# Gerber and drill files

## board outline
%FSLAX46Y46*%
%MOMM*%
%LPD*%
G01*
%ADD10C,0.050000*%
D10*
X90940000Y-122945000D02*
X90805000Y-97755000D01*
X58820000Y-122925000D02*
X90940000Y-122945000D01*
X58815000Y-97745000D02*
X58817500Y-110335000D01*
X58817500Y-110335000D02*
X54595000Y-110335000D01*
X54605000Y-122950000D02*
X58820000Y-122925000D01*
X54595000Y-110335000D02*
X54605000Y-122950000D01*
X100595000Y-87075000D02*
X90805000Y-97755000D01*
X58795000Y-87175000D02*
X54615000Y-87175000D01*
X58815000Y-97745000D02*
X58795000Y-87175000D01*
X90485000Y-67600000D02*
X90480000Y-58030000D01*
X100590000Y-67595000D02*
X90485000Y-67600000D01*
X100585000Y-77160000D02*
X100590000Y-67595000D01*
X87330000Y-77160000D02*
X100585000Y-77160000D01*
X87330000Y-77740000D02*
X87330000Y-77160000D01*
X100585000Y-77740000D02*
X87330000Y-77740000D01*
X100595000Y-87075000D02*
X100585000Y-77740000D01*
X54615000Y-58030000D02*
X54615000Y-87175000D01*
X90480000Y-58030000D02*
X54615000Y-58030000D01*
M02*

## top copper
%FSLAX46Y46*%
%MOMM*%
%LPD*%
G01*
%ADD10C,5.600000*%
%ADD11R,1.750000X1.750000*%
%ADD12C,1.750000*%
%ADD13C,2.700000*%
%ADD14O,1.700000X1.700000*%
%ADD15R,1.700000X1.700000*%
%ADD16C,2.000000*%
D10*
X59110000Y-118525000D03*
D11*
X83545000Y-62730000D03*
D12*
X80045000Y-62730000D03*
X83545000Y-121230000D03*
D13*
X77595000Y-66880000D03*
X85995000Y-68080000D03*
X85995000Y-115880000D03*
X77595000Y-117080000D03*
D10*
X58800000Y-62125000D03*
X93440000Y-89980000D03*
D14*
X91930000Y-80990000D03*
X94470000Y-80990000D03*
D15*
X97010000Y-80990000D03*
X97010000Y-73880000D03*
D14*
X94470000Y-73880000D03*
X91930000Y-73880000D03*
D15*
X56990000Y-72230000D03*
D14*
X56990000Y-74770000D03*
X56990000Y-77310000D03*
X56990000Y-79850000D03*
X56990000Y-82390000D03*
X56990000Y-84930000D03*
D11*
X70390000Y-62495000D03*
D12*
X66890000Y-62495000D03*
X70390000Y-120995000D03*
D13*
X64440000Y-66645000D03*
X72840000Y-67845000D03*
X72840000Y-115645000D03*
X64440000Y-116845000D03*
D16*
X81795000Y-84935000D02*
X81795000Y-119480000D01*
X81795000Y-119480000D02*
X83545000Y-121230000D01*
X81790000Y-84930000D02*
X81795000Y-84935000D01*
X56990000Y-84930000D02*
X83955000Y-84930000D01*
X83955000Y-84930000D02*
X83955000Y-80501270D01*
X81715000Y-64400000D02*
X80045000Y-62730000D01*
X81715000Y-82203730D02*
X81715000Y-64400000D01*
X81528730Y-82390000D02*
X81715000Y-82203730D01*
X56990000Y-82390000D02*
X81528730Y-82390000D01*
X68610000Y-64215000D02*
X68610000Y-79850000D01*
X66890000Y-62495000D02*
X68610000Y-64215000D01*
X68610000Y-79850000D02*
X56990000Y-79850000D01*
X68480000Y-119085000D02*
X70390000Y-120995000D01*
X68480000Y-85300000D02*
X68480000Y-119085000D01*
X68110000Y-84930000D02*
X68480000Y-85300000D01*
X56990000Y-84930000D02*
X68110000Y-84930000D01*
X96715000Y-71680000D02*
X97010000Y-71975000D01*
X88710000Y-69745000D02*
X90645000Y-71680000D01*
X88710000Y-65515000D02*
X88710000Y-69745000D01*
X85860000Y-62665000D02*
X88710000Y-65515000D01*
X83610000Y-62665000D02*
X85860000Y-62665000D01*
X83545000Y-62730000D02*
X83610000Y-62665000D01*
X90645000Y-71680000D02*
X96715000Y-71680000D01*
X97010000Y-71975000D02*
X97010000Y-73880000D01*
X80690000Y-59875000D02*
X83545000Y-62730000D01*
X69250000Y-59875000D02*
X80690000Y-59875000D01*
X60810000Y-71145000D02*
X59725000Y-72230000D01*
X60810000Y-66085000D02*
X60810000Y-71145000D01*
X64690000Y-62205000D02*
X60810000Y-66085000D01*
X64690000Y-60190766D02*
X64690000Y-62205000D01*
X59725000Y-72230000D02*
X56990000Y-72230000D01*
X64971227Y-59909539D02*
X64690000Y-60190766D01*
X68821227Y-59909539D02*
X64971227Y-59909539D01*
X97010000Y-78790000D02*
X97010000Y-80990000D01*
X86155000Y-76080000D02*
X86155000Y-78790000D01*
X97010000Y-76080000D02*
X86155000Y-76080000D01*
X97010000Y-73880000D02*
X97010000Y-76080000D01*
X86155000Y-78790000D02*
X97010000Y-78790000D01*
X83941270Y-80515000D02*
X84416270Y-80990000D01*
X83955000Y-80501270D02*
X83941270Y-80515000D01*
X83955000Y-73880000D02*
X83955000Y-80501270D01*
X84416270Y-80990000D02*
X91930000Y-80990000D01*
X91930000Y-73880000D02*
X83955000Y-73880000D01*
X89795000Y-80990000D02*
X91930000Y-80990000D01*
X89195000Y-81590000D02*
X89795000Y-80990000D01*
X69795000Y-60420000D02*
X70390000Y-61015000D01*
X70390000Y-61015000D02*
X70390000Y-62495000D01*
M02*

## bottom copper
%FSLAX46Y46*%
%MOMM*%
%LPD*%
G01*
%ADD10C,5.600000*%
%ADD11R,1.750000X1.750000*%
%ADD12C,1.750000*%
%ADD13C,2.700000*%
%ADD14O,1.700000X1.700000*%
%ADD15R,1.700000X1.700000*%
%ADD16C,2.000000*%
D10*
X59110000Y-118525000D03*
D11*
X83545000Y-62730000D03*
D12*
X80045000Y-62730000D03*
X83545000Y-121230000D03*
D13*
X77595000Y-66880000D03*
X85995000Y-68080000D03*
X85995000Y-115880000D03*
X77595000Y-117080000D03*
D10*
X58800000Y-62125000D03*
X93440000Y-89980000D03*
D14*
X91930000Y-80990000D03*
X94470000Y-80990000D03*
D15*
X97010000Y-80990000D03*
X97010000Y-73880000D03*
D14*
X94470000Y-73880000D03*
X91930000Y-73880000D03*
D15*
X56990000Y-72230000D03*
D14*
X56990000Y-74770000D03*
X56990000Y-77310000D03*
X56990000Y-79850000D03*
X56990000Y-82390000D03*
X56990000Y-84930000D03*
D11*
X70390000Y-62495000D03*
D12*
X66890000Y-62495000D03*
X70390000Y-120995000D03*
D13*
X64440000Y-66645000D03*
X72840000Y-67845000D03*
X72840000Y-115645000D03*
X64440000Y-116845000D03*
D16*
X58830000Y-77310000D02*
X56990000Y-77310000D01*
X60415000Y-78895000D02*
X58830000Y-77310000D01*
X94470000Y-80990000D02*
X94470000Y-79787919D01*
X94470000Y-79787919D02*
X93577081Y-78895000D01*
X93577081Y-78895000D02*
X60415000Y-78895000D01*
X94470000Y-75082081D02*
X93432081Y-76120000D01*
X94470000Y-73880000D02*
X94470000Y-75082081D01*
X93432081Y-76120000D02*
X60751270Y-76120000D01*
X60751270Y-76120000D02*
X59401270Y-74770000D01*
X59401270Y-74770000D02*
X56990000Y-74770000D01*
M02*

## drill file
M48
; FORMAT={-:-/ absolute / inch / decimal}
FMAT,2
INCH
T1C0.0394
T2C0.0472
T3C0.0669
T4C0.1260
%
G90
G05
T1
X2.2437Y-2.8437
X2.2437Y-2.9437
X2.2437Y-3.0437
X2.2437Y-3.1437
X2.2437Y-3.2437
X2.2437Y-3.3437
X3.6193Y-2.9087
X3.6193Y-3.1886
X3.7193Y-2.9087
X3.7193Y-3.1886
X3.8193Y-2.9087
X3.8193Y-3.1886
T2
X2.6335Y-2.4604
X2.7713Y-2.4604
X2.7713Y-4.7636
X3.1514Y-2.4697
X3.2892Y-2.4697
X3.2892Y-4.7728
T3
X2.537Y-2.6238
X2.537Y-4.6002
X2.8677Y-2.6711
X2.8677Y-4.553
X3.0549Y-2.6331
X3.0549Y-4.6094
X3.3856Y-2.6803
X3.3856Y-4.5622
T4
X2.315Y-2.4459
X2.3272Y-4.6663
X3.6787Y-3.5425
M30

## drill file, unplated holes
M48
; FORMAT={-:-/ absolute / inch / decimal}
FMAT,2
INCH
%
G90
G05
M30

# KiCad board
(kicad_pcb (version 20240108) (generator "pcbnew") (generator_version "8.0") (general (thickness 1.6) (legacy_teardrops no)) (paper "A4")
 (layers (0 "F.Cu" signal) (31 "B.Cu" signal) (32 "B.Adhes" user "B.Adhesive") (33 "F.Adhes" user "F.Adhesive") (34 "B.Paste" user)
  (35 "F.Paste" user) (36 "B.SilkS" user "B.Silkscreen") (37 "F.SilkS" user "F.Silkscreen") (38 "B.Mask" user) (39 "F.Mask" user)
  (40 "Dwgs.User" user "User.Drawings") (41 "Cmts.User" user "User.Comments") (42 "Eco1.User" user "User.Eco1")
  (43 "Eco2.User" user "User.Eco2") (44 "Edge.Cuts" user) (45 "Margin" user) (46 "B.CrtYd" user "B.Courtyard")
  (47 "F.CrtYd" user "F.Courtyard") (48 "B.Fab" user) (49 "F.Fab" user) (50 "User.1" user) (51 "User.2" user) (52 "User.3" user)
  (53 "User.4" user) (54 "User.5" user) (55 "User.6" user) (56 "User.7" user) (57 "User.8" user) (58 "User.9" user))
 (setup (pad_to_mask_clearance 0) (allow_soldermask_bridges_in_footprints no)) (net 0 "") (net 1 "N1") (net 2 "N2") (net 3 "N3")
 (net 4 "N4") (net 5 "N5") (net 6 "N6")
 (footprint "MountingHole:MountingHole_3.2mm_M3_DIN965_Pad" (layer "F.Cu") (at 93.44 89.98)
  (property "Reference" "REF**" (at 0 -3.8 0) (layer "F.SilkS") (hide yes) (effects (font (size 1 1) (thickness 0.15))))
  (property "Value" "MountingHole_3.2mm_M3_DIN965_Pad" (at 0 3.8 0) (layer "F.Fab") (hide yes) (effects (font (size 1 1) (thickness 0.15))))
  (pad "1" thru_hole circle (at 0 0) (size 5.6 5.6) (drill 3.2) (layers "*.Cu" "*.Mask") (remove_unused_layers no)))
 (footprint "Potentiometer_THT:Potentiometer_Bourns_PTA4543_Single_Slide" (layer "F.Cu") (at 83.545 62.73 -90)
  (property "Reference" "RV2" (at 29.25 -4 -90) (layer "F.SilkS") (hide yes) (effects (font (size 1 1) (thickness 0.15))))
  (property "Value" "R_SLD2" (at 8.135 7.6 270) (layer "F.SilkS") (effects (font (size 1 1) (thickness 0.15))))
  (pad "1" thru_hole rect (at 0 0 270) (size 1.75 1.75) (drill 1.2) (layers "*.Cu" "*.Mask") (remove_unused_layers no) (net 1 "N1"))
  (pad "2" thru_hole circle (at 0 3.5 270) (size 1.75 1.75) (drill 1.2) (layers "*.Cu" "*.Mask") (remove_unused_layers no) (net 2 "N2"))
  (pad "3" thru_hole circle (at 58.5 0 270) (size 1.75 1.75) (drill 1.2) (layers "*.Cu" "*.Mask") (remove_unused_layers no) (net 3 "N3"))
  (pad "MP" thru_hole circle (at 4.15 5.95 270) (size 2.7 2.7) (drill 1.7) (layers "*.Cu" "*.Mask") (remove_unused_layers no))
  (pad "MP" thru_hole circle (at 5.35 -2.45 270) (size 2.7 2.7) (drill 1.7) (layers "*.Cu" "*.Mask") (remove_unused_layers no))
  (pad "MP" thru_hole circle (at 53.15 -2.45 270) (size 2.7 2.7) (drill 1.7) (layers "*.Cu" "*.Mask") (remove_unused_layers no))
  (pad "MP" thru_hole circle (at 54.35 5.95 270) (size 2.7 2.7) (drill 1.7) (layers "*.Cu" "*.Mask") (remove_unused_layers no)))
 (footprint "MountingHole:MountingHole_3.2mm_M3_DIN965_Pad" (layer "F.Cu") (at 58.8 62.125)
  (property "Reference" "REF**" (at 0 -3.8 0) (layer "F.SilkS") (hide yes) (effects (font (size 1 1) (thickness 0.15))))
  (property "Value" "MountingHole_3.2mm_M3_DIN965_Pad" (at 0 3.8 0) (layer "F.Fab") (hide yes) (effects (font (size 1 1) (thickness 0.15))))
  (pad "1" thru_hole circle (at 0 0) (size 5.6 5.6) (drill 3.2) (layers "*.Cu" "*.Mask") (remove_unused_layers no)))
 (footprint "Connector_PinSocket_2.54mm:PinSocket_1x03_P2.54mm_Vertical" (layer "F.Cu") (at 97.01 73.88 -90)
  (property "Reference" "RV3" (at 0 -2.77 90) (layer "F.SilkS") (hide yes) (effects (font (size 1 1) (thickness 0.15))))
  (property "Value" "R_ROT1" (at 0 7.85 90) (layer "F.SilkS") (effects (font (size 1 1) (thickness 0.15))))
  (pad "1" thru_hole rect (at 0 0 270) (size 1.7 1.7) (drill 1) (layers "*.Cu" "*.Mask") (remove_unused_layers no) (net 1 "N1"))
  (pad "2" thru_hole oval (at 0 2.54 270) (size 1.7 1.7) (drill 1) (layers "*.Cu" "*.Mask") (remove_unused_layers no) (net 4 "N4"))
  (pad "3" thru_hole oval (at 0 5.08 270) (size 1.7 1.7) (drill 1) (layers "*.Cu" "*.Mask") (remove_unused_layers no) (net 3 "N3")))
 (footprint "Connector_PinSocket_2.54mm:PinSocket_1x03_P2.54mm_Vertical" (layer "F.Cu") (at 97.01 80.99 -90)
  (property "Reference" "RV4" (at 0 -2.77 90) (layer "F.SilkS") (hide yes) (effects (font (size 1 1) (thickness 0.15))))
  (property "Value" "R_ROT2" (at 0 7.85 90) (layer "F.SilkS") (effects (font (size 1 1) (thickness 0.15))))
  (pad "1" thru_hole rect (at 0 0 270) (size 1.7 1.7) (drill 1) (layers "*.Cu" "*.Mask") (remove_unused_layers no) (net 1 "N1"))
  (pad "2" thru_hole oval (at 0 2.54 270) (size 1.7 1.7) (drill 1) (layers "*.Cu" "*.Mask") (remove_unused_layers no) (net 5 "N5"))
  (pad "3" thru_hole oval (at 0 5.08 270) (size 1.7 1.7) (drill 1) (layers "*.Cu" "*.Mask") (remove_unused_layers no) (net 3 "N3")))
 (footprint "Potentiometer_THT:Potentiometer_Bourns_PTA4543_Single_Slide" (layer "F.Cu") (at 70.39 62.495 -90)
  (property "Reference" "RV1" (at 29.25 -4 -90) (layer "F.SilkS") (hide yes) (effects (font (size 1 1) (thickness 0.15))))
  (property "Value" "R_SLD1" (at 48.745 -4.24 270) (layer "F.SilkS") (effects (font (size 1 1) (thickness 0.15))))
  (pad "1" thru_hole rect (at 0 0 270) (size 1.75 1.75) (drill 1.2) (layers "*.Cu" "*.Mask") (remove_unused_layers no) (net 1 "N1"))
  (pad "2" thru_hole circle (at 0 3.5 270) (size 1.75 1.75) (drill 1.2) (layers "*.Cu" "*.Mask") (remove_unused_layers no) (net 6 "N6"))
  (pad "3" thru_hole circle (at 58.5 0 270) (size 1.75 1.75) (drill 1.2) (layers "*.Cu" "*.Mask") (remove_unused_layers no) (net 3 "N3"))
  (pad "MP" thru_hole circle (at 4.15 5.95 270) (size 2.7 2.7) (drill 1.7) (layers "*.Cu" "*.Mask") (remove_unused_layers no))
  (pad "MP" thru_hole circle (at 5.35 -2.45 270) (size 2.7 2.7) (drill 1.7) (layers "*.Cu" "*.Mask") (remove_unused_layers no))
  (pad "MP" thru_hole circle (at 53.15 -2.45 270) (size 2.7 2.7) (drill 1.7) (layers "*.Cu" "*.Mask") (remove_unused_layers no))
  (pad "MP" thru_hole circle (at 54.35 5.95 270) (size 2.7 2.7) (drill 1.7) (layers "*.Cu" "*.Mask") (remove_unused_layers no)))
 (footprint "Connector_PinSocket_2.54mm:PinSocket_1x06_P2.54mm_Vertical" (layer "F.Cu") (at 56.99 72.23)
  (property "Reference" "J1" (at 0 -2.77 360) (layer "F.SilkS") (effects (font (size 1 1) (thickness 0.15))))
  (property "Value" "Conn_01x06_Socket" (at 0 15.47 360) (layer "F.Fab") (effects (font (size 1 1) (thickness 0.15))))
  (pad "1" thru_hole rect (at 0 0) (size 1.7 1.7) (drill 1) (layers "*.Cu" "*.Mask") (remove_unused_layers no) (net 1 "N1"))
  (pad "2" thru_hole oval (at 0 2.54) (size 1.7 1.7) (drill 1) (layers "*.Cu" "*.Mask") (remove_unused_layers no) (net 4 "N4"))
  (pad "3" thru_hole oval (at 0 5.08) (size 1.7 1.7) (drill 1) (layers "*.Cu" "*.Mask") (remove_unused_layers no) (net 5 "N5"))
  (pad "4" thru_hole oval (at 0 7.62) (size 1.7 1.7) (drill 1) (layers "*.Cu" "*.Mask") (remove_unused_layers no) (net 6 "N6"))
  (pad "5" thru_hole oval (at 0 10.16) (size 1.7 1.7) (drill 1) (layers "*.Cu" "*.Mask") (remove_unused_layers no) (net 2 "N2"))
  (pad "6" thru_hole oval (at 0 12.7) (size 1.7 1.7) (drill 1) (layers "*.Cu" "*.Mask") (remove_unused_layers no) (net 3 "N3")))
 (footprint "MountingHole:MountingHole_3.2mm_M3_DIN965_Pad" (layer "F.Cu") (at 59.11 118.525)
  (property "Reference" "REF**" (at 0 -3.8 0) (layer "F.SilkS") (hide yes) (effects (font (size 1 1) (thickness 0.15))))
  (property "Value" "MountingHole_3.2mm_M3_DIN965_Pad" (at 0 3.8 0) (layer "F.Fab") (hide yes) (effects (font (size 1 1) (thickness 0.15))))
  (pad "1" thru_hole circle (at 0 0) (size 5.6 5.6) (drill 3.2) (layers "*.Cu" "*.Mask") (remove_unused_layers no)))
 (gr_line (start 54.595 110.335) (end 54.605 122.95) (stroke (width 0.05) (type default)) (layer "Edge.Cuts"))
 (gr_line (start 90.48 58.03) (end 54.615 58.03) (stroke (width 0.05) (type default)) (layer "Edge.Cuts"))
 (gr_line (start 58.8175 110.335) (end 54.595 110.335) (stroke (width 0.05) (type default)) (layer "Edge.Cuts"))
 (gr_line (start 58.795 87.175) (end 54.615 87.175) (stroke (width 0.05) (type default)) (layer "Edge.Cuts"))
 (gr_line (start 58.82 122.925) (end 90.94 122.945) (stroke (width 0.05) (type default)) (layer "Edge.Cuts"))
 (gr_line (start 90.485 67.6) (end 90.48 58.03) (stroke (width 0.05) (type default)) (layer "Edge.Cuts"))
 (gr_line (start 100.595 87.075) (end 100.585 77.74) (stroke (width 0.05) (type default)) (layer "Edge.Cuts"))
 (gr_line (start 100.585 77.16) (end 100.59 67.595) (stroke (width 0.05) (type default)) (layer "Edge.Cuts"))
 (gr_line (start 100.59 67.595) (end 90.485 67.6) (stroke (width 0.05) (type default)) (layer "Edge.Cuts"))
 (gr_line (start 87.33 77.74) (end 87.33 77.16) (stroke (width 0.05) (type default)) (layer "Edge.Cuts"))
 (gr_line (start 100.595 87.075) (end 90.805 97.755) (stroke (width 0.05) (type default)) (layer "Edge.Cuts"))
 (gr_line (start 54.605 122.95) (end 58.82 122.925) (stroke (width 0.05) (type default)) (layer "Edge.Cuts"))
 (gr_line (start 58.815 97.745) (end 58.795 87.175) (stroke (width 0.05) (type default)) (layer "Edge.Cuts"))
 (gr_line (start 90.94 122.945) (end 90.805 97.755) (stroke (width 0.05) (type default)) (layer "Edge.Cuts"))
 (gr_line (start 87.33 77.16) (end 100.585 77.16) (stroke (width 0.05) (type default)) (layer "Edge.Cuts"))
 (gr_line (start 58.815 97.745) (end 58.8175 110.335) (stroke (width 0.05) (type default)) (layer "Edge.Cuts"))
 (gr_line (start 54.615 58.03) (end 54.615 87.175) (stroke (width 0.05) (type default)) (layer "Edge.Cuts"))
 (gr_line (start 100.585 77.74) (end 87.33 77.74) (stroke (width 0.05) (type default)) (layer "Edge.Cuts"))
 (segment (start 56.99 84.93) (end 83.955 84.93) (width 2) (layer "F.Cu") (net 3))
 (segment (start 89.195 81.59) (end 89.795 80.99) (width 2) (layer "F.Cu") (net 3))
 (segment (start 81.79 84.93) (end 81.795 84.935) (width 2) (layer "F.Cu") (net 3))
 (segment (start 81.795 84.935) (end 81.795 119.48) (width 2) (layer "F.Cu") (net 3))
 (segment (start 83.955 73.88) (end 83.955 80.50127) (width 2) (layer "F.Cu") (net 3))
 (segment (start 84.41627 80.99) (end 91.93 80.99) (width 2) (layer "F.Cu") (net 3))
 (segment (start 89.795 80.99) (end 91.93 80.99) (width 2) (layer "F.Cu") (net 3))
 (segment (start 68.48 119.085) (end 70.39 120.995) (width 2) (layer "F.Cu") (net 3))
 (segment (start 81.795 119.48) (end 83.545 121.23) (width 2) (layer "F.Cu") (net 3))
 (segment (start 68.48 85.3) (end 68.48 119.085) (width 2) (layer "F.Cu") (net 3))
 (segment (start 83.955 84.93) (end 83.955 80.50127) (width 2) (layer "F.Cu") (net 3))
 (segment (start 68.11 84.93) (end 68.48 85.3) (width 2) (layer "F.Cu") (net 3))
 (segment (start 91.93 73.88) (end 83.955 73.88) (width 2) (layer "F.Cu") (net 3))
 (segment (start 83.955 80.50127) (end 83.94127 80.515) (width 2) (layer "F.Cu") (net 3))
 (segment (start 56.99 84.93) (end 68.11 84.93) (width 2) (layer "F.Cu") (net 3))
 (segment (start 83.94127 80.515) (end 84.41627 80.99) (width 2) (layer "F.Cu") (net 3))
 (segment (start 69.25 59.875) (end 80.69 59.875) (width 2) (layer "F.Cu") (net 1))
 (segment (start 85.86 62.665) (end 88.71 65.515) (width 2) (layer "F.Cu") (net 1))
 (segment (start 70.39 61.015) (end 70.39 62.495) (width 2) (layer "F.Cu") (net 1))
 (segment (start 83.61 62.665) (end 85.86 62.665) (width 2) (layer "F.Cu") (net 1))
 (segment (start 64.69 62.205) (end 60.81 66.085) (width 2) (layer "F.Cu") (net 1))
 (segment (start 68.821227 59.909539) (end 64.971227 59.909539) (width 2) (layer "F.Cu") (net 1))
 (segment (start 88.71 65.515) (end 88.71 69.745) (width 2) (layer "F.Cu") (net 1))
 (segment (start 59.725 72.23) (end 56.99 72.23) (width 2) (layer "F.Cu") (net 1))
 (segment (start 80.69 59.875) (end 83.545 62.73) (width 2) (layer "F.Cu") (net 1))
 (segment (start 60.81 66.085) (end 60.81 71.145) (width 2) (layer "F.Cu") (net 1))
 (segment (start 86.155 78.79) (end 97.01 78.79) (width 2) (layer "F.Cu") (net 1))
 (segment (start 88.71 69.745) (end 90.645 71.68) (width 2) (layer "F.Cu") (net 1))
 (segment (start 90.645 71.68) (end 96.715 71.68) (width 2) (layer "F.Cu") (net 1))
 (segment (start 64.971227 59.909539) (end 64.69 60.190766) (width 2) (layer "F.Cu") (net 1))
 (segment (start 83.545 62.73) (end 83.61 62.665) (width 2) (layer "F.Cu") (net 1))
 (segment (start 97.01 71.975) (end 97.01 73.88) (width 2) (layer "F.Cu") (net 1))
 (segment (start 97.01 76.08) (end 86.155 76.08) (width 2) (layer "F.Cu") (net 1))
 (segment (start 69.795 60.42) (end 70.39 61.015) (width 2) (layer "F.Cu") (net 1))
 (segment (start 96.715 71.68) (end 97.01 71.975) (width 2) (layer "F.Cu") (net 1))
 (segment (start 97.01 73.88) (end 97.01 76.08) (width 2) (layer "F.Cu") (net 1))
 (segment (start 86.155 76.08) (end 86.155 78.79) (width 2) (layer "F.Cu") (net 1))
 (segment (start 97.01 78.79) (end 97.01 80.99) (width 2) (layer "F.Cu") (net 1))
 (segment (start 60.81 71.145) (end 59.725 72.23) (width 2) (layer "F.Cu") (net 1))
 (segment (start 64.69 60.190766) (end 64.69 62.205) (width 2) (layer "F.Cu") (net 1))
 (segment (start 81.52873 82.39) (end 81.715 82.20373) (width 2) (layer "F.Cu") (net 2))
 (segment (start 56.99 82.39) (end 81.52873 82.39) (width 2) (layer "F.Cu") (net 2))
 (segment (start 81.715 64.4) (end 80.045 62.73) (width 2) (layer "F.Cu") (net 2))
 (segment (start 81.715 82.20373) (end 81.715 64.4) (width 2) (layer "F.Cu") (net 2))
 (segment (start 68.61 64.215) (end 68.61 79.85) (width 2) (layer "F.Cu") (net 6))
 (segment (start 66.89 62.495) (end 68.61 64.215) (width 2) (layer "F.Cu") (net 6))
 (segment (start 68.61 79.85) (end 56.99 79.85) (width 2) (layer "F.Cu") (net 6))
 (segment (start 94.47 80.99) (end 94.47 79.787919) (width 2) (layer "B.Cu") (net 5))
 (segment (start 94.47 79.787919) (end 93.577081 78.895) (width 2) (layer "B.Cu") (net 5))
 (segment (start 58.83 77.31) (end 56.99 77.31) (width 2) (layer "B.Cu") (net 5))
 (segment (start 93.577081 78.895) (end 60.415 78.895) (width 2) (layer "B.Cu") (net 5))
 (segment (start 60.415 78.895) (end 58.83 77.31) (width 2) (layer "B.Cu") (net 5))
 (segment (start 93.432081 76.12) (end 60.75127 76.12) (width 2) (layer "B.Cu") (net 4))
 (segment (start 60.75127 76.12) (end 59.40127 74.77) (width 2) (layer "B.Cu") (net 4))
 (segment (start 94.47 73.88) (end 94.47 75.082081) (width 2) (layer "B.Cu") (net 4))
 (segment (start 94.47 75.082081) (end 93.432081 76.12) (width 2) (layer "B.Cu") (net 4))
 (segment (start 59.40127 74.77) (end 56.99 74.77) (width 2) (layer "B.Cu") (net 4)))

